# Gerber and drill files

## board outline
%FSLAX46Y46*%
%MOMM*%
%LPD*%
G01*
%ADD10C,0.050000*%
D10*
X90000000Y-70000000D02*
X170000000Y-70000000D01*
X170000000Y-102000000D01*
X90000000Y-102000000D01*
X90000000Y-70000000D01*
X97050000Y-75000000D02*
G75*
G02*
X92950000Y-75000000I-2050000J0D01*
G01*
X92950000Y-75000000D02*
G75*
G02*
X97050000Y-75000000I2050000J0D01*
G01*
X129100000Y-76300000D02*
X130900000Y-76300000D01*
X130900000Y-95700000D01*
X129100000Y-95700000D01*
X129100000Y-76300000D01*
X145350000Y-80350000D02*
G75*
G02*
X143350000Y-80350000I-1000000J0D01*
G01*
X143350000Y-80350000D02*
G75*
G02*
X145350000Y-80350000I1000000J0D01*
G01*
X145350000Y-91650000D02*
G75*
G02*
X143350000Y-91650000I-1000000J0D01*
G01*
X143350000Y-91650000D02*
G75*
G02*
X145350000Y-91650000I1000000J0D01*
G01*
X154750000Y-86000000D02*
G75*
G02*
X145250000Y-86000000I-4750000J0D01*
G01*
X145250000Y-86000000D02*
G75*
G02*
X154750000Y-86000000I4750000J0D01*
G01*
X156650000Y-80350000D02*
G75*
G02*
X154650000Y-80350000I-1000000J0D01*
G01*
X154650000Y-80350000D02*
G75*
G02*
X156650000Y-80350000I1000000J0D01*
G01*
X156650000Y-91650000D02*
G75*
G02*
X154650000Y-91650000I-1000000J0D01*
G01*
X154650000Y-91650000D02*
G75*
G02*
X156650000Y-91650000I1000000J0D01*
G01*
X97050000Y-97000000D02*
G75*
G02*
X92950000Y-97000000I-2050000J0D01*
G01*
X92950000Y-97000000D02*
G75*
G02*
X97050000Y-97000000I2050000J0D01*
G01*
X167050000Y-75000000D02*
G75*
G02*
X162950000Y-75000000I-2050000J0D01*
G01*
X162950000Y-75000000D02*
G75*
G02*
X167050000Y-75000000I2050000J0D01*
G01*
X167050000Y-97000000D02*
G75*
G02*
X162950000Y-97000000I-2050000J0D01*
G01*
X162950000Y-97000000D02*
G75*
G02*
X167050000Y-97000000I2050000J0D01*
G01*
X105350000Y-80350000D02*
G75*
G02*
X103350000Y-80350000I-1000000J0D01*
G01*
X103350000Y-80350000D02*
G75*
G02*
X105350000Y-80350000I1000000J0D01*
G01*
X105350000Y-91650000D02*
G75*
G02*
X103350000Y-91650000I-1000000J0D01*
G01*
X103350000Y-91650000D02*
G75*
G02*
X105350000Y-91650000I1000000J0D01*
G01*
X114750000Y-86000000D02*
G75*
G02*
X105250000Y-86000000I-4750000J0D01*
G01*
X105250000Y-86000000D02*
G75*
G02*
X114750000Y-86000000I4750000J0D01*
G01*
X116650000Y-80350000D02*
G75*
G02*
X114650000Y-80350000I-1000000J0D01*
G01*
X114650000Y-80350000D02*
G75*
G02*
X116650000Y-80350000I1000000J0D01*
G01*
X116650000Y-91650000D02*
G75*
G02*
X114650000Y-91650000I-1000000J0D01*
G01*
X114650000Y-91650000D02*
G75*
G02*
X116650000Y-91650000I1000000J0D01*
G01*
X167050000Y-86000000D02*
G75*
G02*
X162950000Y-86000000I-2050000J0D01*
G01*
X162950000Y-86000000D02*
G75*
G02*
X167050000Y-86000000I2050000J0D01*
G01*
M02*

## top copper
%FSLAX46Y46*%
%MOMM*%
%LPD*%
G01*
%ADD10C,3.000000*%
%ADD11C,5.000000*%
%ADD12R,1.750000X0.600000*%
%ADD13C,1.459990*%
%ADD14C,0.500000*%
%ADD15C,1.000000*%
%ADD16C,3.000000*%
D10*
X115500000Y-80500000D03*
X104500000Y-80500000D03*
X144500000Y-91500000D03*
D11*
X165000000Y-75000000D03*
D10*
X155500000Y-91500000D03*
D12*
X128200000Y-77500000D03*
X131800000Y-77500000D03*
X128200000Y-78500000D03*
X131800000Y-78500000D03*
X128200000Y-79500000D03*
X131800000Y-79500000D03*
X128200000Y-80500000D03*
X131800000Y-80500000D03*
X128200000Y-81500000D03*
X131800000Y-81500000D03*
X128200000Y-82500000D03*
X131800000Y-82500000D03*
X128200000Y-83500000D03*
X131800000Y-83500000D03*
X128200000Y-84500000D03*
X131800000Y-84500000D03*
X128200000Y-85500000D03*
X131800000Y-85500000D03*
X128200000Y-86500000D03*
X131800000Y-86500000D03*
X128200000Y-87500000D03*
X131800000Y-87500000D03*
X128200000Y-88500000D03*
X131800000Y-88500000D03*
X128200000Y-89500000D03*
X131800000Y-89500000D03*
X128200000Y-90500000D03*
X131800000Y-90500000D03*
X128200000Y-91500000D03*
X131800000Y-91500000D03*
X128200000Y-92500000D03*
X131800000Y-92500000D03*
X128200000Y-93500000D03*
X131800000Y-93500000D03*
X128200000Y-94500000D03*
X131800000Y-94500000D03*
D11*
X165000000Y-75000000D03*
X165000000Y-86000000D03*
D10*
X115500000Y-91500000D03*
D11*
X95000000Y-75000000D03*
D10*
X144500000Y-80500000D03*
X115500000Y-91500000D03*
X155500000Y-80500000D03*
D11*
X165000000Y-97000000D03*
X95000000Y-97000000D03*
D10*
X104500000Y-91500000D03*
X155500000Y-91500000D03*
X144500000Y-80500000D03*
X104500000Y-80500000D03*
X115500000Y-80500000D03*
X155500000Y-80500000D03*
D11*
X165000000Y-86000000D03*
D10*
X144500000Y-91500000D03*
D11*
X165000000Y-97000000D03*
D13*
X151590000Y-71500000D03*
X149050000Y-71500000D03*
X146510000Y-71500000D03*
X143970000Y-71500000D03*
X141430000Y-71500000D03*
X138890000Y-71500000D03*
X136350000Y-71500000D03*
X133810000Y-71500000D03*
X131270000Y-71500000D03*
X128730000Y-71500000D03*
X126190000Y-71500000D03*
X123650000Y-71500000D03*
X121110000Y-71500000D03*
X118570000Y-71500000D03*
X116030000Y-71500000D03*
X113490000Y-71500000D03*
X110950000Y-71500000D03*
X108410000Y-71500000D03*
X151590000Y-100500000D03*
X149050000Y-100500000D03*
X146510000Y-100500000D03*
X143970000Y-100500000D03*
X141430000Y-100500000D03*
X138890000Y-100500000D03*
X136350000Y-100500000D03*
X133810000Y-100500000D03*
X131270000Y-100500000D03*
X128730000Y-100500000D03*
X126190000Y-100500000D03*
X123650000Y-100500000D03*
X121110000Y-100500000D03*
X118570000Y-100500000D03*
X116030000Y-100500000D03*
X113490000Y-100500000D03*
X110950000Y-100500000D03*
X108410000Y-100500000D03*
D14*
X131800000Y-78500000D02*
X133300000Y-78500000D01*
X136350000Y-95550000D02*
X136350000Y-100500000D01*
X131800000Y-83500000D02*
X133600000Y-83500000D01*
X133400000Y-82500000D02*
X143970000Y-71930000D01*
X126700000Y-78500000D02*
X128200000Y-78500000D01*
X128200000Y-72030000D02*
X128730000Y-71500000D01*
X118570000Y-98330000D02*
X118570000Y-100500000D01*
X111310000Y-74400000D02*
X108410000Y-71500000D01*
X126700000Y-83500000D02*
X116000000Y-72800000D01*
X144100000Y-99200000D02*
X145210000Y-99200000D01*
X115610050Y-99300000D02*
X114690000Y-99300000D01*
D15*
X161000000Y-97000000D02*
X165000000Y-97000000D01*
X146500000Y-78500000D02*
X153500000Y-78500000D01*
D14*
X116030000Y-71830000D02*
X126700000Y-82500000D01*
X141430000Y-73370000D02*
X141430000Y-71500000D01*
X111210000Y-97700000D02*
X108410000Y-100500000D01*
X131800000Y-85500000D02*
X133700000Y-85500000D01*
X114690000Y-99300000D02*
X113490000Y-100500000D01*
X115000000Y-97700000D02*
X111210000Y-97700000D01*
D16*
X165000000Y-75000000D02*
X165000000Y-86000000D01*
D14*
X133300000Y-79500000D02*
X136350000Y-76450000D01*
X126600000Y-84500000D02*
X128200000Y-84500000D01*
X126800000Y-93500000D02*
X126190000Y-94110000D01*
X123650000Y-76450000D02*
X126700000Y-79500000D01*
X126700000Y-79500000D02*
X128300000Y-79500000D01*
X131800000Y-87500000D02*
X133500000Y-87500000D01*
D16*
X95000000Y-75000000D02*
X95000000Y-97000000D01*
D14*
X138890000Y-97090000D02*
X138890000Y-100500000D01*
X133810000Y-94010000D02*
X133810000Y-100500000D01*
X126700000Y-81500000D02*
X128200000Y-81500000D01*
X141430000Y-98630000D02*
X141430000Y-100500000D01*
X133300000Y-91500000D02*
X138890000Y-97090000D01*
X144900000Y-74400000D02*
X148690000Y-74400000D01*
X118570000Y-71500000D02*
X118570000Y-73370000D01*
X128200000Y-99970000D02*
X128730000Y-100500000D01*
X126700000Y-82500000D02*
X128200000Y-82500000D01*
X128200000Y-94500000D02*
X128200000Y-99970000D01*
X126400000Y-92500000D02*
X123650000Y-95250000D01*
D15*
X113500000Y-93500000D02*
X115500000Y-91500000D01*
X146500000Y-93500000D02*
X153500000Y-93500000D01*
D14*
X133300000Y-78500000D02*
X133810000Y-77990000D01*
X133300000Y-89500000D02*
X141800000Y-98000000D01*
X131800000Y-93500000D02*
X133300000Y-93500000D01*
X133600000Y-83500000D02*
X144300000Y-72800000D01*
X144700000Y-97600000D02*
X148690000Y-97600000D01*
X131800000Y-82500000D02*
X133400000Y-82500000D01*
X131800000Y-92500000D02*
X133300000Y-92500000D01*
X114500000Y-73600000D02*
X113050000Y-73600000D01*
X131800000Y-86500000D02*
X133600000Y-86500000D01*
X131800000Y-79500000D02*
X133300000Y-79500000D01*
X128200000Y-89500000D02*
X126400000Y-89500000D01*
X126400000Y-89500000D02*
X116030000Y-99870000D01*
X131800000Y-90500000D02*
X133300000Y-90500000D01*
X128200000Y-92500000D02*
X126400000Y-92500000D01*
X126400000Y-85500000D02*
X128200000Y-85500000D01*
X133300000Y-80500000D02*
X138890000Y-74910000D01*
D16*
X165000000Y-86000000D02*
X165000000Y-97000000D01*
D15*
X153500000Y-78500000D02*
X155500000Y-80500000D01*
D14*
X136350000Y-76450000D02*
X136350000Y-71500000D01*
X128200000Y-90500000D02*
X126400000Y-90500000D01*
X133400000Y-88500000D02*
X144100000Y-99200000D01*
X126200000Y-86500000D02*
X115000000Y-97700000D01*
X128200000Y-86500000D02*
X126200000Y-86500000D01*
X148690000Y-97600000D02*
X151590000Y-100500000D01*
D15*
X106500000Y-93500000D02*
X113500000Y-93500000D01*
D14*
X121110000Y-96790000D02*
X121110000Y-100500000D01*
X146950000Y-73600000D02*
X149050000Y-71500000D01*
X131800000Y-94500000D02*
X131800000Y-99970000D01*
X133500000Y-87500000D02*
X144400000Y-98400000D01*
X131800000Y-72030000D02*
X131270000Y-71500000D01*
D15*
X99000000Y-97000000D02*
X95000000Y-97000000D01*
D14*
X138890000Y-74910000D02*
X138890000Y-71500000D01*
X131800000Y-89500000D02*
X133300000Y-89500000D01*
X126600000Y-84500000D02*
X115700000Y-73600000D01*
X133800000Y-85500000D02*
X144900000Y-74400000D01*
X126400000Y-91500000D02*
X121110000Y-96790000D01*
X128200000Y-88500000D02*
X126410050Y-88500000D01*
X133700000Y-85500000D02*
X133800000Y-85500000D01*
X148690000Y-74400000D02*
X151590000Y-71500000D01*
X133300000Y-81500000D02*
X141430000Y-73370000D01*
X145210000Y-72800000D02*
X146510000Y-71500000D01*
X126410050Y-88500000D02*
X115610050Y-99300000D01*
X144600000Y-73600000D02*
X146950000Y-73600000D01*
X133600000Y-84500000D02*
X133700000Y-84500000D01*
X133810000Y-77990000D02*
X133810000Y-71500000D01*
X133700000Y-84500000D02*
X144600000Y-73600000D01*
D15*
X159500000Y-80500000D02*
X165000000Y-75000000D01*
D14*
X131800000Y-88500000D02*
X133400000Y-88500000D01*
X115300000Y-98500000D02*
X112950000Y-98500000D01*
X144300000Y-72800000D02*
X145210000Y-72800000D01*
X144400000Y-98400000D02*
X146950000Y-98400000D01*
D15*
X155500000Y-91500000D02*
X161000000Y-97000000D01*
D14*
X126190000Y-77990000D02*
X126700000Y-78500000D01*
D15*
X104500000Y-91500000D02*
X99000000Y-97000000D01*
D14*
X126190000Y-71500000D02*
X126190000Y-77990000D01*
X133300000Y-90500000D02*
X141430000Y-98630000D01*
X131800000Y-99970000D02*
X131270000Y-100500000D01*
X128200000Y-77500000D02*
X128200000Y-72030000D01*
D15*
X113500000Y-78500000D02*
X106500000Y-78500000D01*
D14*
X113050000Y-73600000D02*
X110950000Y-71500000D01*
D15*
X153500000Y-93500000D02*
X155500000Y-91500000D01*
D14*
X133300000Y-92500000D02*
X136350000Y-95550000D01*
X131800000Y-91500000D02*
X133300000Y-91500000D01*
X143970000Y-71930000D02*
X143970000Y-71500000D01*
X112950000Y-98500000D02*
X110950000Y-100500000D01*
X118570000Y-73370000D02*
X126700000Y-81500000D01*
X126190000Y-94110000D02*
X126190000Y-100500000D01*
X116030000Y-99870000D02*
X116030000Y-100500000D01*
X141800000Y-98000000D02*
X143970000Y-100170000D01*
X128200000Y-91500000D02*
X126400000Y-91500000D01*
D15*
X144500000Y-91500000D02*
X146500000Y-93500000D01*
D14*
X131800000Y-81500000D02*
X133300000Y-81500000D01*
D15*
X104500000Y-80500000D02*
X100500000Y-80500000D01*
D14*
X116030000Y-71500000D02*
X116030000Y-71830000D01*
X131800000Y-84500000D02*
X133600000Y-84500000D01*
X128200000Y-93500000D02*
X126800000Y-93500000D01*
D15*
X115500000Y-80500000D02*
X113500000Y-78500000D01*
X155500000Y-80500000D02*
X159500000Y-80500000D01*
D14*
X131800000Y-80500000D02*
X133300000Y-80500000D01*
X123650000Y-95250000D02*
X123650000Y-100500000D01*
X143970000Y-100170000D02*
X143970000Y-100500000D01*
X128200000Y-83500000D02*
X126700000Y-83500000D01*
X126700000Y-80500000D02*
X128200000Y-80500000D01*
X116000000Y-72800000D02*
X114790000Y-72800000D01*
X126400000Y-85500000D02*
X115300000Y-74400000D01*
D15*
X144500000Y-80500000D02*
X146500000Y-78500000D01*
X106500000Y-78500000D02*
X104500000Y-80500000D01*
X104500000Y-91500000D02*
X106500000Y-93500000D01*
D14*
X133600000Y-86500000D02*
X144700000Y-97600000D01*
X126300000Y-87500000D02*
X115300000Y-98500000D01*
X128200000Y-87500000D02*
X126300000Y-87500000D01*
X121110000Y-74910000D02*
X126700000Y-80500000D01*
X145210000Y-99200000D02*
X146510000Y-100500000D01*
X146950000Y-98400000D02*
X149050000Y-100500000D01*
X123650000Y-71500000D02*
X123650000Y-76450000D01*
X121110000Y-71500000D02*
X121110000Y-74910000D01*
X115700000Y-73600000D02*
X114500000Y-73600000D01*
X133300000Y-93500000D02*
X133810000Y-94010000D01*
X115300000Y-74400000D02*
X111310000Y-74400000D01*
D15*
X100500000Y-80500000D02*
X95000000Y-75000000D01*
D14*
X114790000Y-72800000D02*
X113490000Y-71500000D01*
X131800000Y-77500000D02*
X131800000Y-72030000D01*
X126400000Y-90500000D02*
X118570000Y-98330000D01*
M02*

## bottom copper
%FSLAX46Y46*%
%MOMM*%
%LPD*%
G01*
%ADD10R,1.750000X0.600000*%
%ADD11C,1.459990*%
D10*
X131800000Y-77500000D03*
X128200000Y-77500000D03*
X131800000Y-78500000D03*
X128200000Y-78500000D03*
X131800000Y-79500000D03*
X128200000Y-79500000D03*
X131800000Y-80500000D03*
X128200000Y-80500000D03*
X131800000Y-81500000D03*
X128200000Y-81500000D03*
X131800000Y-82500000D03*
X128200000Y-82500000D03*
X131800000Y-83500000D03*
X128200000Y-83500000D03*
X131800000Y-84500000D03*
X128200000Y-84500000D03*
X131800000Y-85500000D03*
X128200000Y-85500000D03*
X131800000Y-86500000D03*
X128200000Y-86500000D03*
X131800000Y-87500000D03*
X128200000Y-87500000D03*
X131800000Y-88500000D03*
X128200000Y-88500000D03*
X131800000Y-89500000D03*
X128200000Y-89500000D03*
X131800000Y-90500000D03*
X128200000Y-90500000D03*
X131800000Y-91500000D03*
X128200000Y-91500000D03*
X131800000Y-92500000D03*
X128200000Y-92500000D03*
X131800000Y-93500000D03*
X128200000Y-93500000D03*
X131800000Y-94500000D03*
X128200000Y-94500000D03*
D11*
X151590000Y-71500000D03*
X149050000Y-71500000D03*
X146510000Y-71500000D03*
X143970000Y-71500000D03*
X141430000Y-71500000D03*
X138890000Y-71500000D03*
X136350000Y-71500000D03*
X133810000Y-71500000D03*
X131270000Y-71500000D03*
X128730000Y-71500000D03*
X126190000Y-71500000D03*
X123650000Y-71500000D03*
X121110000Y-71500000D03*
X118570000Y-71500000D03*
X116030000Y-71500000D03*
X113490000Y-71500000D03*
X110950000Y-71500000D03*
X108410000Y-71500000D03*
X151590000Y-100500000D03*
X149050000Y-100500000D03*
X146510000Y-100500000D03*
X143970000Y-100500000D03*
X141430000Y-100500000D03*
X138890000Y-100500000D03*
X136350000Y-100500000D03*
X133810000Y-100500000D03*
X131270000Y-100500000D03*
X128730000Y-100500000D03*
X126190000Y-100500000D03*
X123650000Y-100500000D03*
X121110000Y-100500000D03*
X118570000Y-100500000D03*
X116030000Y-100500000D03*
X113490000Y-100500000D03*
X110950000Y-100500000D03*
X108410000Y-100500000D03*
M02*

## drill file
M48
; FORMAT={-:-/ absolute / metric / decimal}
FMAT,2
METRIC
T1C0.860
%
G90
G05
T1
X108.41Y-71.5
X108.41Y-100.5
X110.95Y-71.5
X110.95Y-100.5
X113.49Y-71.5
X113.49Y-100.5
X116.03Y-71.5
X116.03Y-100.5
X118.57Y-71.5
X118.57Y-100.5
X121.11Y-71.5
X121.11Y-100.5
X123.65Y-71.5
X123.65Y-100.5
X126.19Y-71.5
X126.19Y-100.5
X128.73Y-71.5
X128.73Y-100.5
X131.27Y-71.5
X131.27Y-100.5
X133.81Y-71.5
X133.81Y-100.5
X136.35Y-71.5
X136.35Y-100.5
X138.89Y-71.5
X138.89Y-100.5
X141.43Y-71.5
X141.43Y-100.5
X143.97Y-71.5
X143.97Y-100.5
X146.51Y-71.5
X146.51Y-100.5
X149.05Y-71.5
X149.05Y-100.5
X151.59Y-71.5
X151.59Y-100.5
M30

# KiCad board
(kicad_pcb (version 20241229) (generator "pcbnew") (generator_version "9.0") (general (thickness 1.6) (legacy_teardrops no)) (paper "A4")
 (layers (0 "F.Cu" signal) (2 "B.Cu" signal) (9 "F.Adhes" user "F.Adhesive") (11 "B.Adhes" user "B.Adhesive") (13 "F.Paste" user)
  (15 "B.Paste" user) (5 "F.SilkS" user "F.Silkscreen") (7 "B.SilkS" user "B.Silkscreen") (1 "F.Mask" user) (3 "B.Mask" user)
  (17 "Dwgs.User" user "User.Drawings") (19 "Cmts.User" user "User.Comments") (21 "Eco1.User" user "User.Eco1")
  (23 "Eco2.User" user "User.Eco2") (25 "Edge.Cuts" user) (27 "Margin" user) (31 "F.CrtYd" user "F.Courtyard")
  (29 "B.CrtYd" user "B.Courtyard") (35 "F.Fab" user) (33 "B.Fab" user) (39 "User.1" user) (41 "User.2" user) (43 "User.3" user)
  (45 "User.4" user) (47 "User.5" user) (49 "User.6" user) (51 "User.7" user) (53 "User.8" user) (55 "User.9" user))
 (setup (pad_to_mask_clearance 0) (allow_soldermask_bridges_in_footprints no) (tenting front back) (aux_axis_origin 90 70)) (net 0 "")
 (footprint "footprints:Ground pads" (layer "F.Cu") (at 115.5 80.5)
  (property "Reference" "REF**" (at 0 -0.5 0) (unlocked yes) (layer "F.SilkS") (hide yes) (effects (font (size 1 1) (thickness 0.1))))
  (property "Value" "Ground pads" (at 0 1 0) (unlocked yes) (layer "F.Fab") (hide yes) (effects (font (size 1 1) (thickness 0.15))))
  (pad "1" smd circle (at 0 0) (size 3 3) (layers "F.Cu" "F.Mask" "F.Paste")))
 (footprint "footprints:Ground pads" (layer "F.Cu") (at 104.5 80.5)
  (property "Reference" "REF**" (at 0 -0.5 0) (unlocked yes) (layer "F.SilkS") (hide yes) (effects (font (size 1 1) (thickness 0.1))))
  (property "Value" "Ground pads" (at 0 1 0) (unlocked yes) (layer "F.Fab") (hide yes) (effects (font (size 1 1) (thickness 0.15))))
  (pad "1" smd circle (at 0 0) (size 3 3) (layers "F.Cu" "F.Mask" "F.Paste")))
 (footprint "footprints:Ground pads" (layer "F.Cu") (at 144.5 91.5)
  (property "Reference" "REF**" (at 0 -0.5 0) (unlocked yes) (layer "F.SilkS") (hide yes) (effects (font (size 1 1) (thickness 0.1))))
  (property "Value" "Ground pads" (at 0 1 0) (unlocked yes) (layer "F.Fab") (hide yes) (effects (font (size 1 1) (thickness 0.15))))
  (pad "1" smd circle (at 0 0) (size 3 3) (layers "F.Cu" "F.Mask" "F.Paste")))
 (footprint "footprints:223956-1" (layer "F.Cu") (at 95 75)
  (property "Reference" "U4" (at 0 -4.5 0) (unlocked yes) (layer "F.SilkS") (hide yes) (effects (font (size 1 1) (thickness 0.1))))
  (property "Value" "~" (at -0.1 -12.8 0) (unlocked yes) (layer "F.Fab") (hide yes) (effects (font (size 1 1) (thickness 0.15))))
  (fp_circle (center 0 0) (end 0 2.05) (stroke (width 0.05) (type default)) (fill no) (layer "Edge.Cuts")))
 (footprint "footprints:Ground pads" (layer "F.Cu") (at 165 75)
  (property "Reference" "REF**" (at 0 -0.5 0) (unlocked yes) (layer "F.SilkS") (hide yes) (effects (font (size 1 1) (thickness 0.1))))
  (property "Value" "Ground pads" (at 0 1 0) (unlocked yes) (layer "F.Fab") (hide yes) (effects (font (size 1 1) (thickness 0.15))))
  (pad "1" smd circle (at 0 0) (size 5 5) (layers "F.Cu" "F.Mask" "F.Paste")))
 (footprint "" (layer "F.Cu") (at 155.5 91.5)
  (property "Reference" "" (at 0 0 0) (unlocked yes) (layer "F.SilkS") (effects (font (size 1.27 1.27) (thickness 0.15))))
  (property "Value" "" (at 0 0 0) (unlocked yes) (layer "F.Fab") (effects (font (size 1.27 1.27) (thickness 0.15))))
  (pad "1" smd circle (at 0 0) (size 3 3) (layers "F.Cu" "F.Mask" "F.Paste")))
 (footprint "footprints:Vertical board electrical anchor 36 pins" (layer "F.Cu") (at 130 86)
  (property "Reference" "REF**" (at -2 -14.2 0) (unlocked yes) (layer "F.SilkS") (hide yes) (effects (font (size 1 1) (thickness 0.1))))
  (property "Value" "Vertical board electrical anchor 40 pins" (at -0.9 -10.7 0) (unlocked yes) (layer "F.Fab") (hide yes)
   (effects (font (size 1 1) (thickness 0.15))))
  (fp_rect (start -0.9 -9.7) (end 0.9 9.7) (stroke (width 0.05) (type default)) (fill no) (layer "Edge.Cuts"))
  (pad "01A" smd rect (at -1.8 -8.5 90) (size 0.6 1.75) (layers "F.Cu" "F.Mask" "F.Paste") (solder_mask_margin 0.102))
  (pad "01A" smd rect (at 1.8 -8.5 90) (size 0.6 1.75) (layers "F.Cu" "F.Mask" "F.Paste") (solder_mask_margin 0.102))
  (pad "02A" smd rect (at -1.8 -7.5 90) (size 0.6 1.75) (layers "F.Cu" "F.Mask" "F.Paste") (solder_mask_margin 0.102))
  (pad "02A" smd rect (at 1.8 -7.5 90) (size 0.6 1.75) (layers "F.Cu" "F.Mask" "F.Paste") (solder_mask_margin 0.102))
  (pad "03A" smd rect (at -1.8 -6.5 90) (size 0.6 1.75) (layers "F.Cu" "F.Mask" "F.Paste") (solder_mask_margin 0.102))
  (pad "03A" smd rect (at 1.8 -6.5 90) (size 0.6 1.75) (layers "F.Cu" "F.Mask" "F.Paste") (solder_mask_margin 0.102))
  (pad "04A" smd rect (at -1.8 -5.5 90) (size 0.6 1.75) (layers "F.Cu" "F.Mask" "F.Paste") (solder_mask_margin 0.102))
  (pad "04A" smd rect (at 1.8 -5.5 90) (size 0.6 1.75) (layers "F.Cu" "F.Mask" "F.Paste") (solder_mask_margin 0.102))
  (pad "05A" smd rect (at -1.8 -4.5 90) (size 0.6 1.75) (layers "F.Cu" "F.Mask" "F.Paste") (solder_mask_margin 0.102))
  (pad "05A" smd rect (at 1.8 -4.5 90) (size 0.6 1.75) (layers "F.Cu" "F.Mask" "F.Paste") (solder_mask_margin 0.102))
  (pad "06A" smd rect (at -1.8 -3.5 90) (size 0.6 1.75) (layers "F.Cu" "F.Mask" "F.Paste") (solder_mask_margin 0.102))
  (pad "06A" smd rect (at 1.8 -3.5 90) (size 0.6 1.75) (layers "F.Cu" "F.Mask" "F.Paste") (solder_mask_margin 0.102))
  (pad "07A" smd rect (at -1.8 -2.5 90) (size 0.6 1.75) (layers "F.Cu" "F.Mask" "F.Paste") (solder_mask_margin 0.102))
  (pad "07A" smd rect (at 1.8 -2.5 90) (size 0.6 1.75) (layers "F.Cu" "F.Mask" "F.Paste") (solder_mask_margin 0.102))
  (pad "08A" smd rect (at -1.8 -1.5 90) (size 0.6 1.75) (layers "F.Cu" "F.Mask" "F.Paste") (solder_mask_margin 0.102))
  (pad "08A" smd rect (at 1.8 -1.5 90) (size 0.6 1.75) (layers "F.Cu" "F.Mask" "F.Paste") (solder_mask_margin 0.102))
  (pad "09A" smd rect (at -1.8 -0.5 90) (size 0.6 1.75) (layers "F.Cu" "F.Mask" "F.Paste") (solder_mask_margin 0.102))
  (pad "09A" smd rect (at 1.8 -0.5 90) (size 0.6 1.75) (layers "F.Cu" "F.Mask" "F.Paste") (solder_mask_margin 0.102))
  (pad "10A" smd rect (at -1.8 0.5 90) (size 0.6 1.75) (layers "F.Cu" "F.Mask" "F.Paste") (solder_mask_margin 0.102))
  (pad "10A" smd rect (at 1.8 0.5 90) (size 0.6 1.75) (layers "F.Cu" "F.Mask" "F.Paste") (solder_mask_margin 0.102))
  (pad "11A" smd rect (at -1.8 1.5 90) (size 0.6 1.75) (layers "F.Cu" "F.Mask" "F.Paste") (solder_mask_margin 0.102))
  (pad "11A" smd rect (at 1.8 1.5 90) (size 0.6 1.75) (layers "F.Cu" "F.Mask" "F.Paste") (solder_mask_margin 0.102))
  (pad "12A" smd rect (at -1.8 2.5 90) (size 0.6 1.75) (layers "F.Cu" "F.Mask" "F.Paste") (solder_mask_margin 0.102))
  (pad "12A" smd rect (at 1.8 2.5 90) (size 0.6 1.75) (layers "F.Cu" "F.Mask" "F.Paste") (solder_mask_margin 0.102))
  (pad "13A" smd rect (at -1.8 3.5 90) (size 0.6 1.75) (layers "F.Cu" "F.Mask" "F.Paste") (solder_mask_margin 0.102))
  (pad "13A" smd rect (at 1.8 3.5 90) (size 0.6 1.75) (layers "F.Cu" "F.Mask" "F.Paste") (solder_mask_margin 0.102))
  (pad "14A" smd rect (at -1.8 4.5 90) (size 0.6 1.75) (layers "F.Cu" "F.Mask" "F.Paste") (solder_mask_margin 0.102))
  (pad "14A" smd rect (at 1.8 4.5 90) (size 0.6 1.75) (layers "F.Cu" "F.Mask" "F.Paste") (solder_mask_margin 0.102))
  (pad "15A" smd rect (at -1.8 5.5 90) (size 0.6 1.75) (layers "F.Cu" "F.Mask" "F.Paste") (solder_mask_margin 0.102))
  (pad "15A" smd rect (at 1.8 5.5 90) (size 0.6 1.75) (layers "F.Cu" "F.Mask" "F.Paste") (solder_mask_margin 0.102))
  (pad "16A" smd rect (at -1.8 6.5 90) (size 0.6 1.75) (layers "F.Cu" "F.Mask" "F.Paste") (solder_mask_margin 0.102))
  (pad "16A" smd rect (at 1.8 6.5 90) (size 0.6 1.75) (layers "F.Cu" "F.Mask" "F.Paste") (solder_mask_margin 0.102))
  (pad "17A" smd rect (at -1.8 7.5 90) (size 0.6 1.75) (layers "F.Cu" "F.Mask" "F.Paste") (solder_mask_margin 0.102))
  (pad "17A" smd rect (at 1.8 7.5 90) (size 0.6 1.75) (layers "F.Cu" "F.Mask" "F.Paste") (solder_mask_margin 0.102))
  (pad "18A" smd rect (at -1.8 8.5 90) (size 0.6 1.75) (layers "F.Cu" "F.Mask" "F.Paste") (solder_mask_margin 0.102))
  (pad "18A" smd rect (at 1.8 8.5 90) (size 0.6 1.75) (layers "F.Cu" "F.Mask" "F.Paste") (solder_mask_margin 0.102)))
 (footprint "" (layer "F.Cu") (at 165 75)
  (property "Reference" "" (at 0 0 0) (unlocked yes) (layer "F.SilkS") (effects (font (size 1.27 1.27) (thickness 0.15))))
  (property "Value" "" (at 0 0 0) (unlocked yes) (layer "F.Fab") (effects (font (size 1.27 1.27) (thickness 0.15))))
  (pad "1" smd circle (at 0 0) (size 5 5) (layers "F.Cu" "F.Mask" "F.Paste")))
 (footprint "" (layer "F.Cu") (at 165 86)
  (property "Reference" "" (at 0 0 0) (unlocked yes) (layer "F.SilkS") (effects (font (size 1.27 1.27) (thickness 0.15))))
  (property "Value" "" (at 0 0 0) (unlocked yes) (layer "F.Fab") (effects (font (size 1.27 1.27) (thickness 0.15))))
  (pad "1" smd circle (at 0 0) (size 5 5) (layers "F.Cu" "F.Mask" "F.Paste")))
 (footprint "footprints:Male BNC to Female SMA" (layer "F.Cu") (at 150 86)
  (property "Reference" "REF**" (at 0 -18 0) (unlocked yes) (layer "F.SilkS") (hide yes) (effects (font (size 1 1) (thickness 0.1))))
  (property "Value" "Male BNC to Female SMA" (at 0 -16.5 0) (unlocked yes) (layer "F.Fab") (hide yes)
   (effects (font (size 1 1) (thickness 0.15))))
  (fp_circle (center -5.65 -5.65) (end -5.65 -4.65) (stroke (width 0.05) (type default)) (fill no) (layer "Edge.Cuts"))
  (fp_circle (center -5.65 5.65) (end -5.65 6.65) (stroke (width 0.05) (type default)) (fill no) (layer "Edge.Cuts"))
  (fp_circle (center 0 0) (end 0 -4.75) (stroke (width 0.05) (type default)) (fill no) (layer "Edge.Cuts"))
  (fp_circle (center 5.65 -5.65) (end 5.65 -6.65) (stroke (width 0.05) (type default)) (fill no) (layer "Edge.Cuts"))
  (fp_circle (center 5.65 5.65) (end 4.65 5.65) (stroke (width 0.05) (type default)) (fill no) (layer "Edge.Cuts")))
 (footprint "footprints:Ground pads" (layer "F.Cu") (at 115.5 91.5)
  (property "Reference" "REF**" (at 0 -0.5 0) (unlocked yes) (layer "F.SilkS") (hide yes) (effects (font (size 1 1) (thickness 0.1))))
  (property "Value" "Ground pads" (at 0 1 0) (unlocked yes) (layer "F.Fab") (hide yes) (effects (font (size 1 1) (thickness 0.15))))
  (pad "1" smd circle (at 0 0) (size 3 3) (layers "F.Cu" "F.Mask" "F.Paste")))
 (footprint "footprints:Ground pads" (layer "F.Cu") (at 95 75)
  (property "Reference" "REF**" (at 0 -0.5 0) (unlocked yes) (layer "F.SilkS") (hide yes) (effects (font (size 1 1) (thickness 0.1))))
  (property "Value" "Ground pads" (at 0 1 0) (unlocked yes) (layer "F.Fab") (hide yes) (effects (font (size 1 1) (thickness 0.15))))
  (pad "1" smd circle (at 0 0) (size 5 5) (layers "F.Cu" "F.Mask" "F.Paste")))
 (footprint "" (layer "F.Cu") (at 144.5 80.5)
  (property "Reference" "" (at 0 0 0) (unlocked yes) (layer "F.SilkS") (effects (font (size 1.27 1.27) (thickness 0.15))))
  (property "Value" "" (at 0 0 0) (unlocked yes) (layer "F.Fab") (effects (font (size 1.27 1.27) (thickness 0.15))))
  (pad "1" smd circle (at 0 0) (size 3 3) (layers "F.Cu" "F.Mask" "F.Paste")))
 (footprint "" (layer "F.Cu") (at 115.5 91.5)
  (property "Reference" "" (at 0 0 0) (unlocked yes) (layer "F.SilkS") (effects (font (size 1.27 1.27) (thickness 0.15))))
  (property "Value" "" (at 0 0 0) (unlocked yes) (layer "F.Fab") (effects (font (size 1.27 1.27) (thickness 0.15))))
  (pad "1" smd circle (at 0 0) (size 3 3) (layers "F.Cu" "F.Mask" "F.Paste")))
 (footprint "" (layer "F.Cu") (at 155.5 80.5)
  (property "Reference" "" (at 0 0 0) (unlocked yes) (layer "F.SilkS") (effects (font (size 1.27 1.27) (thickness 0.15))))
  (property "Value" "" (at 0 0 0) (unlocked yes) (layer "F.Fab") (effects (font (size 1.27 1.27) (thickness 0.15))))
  (pad "1" smd circle (at 0 0) (size 3 3) (layers "F.Cu" "F.Mask" "F.Paste")))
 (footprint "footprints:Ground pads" (layer "F.Cu") (at 165 97)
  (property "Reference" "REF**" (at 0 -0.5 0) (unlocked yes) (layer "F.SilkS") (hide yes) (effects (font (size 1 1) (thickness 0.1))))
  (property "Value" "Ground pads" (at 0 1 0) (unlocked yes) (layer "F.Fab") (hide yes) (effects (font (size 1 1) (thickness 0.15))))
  (pad "1" smd circle (at 0 0) (size 5 5) (layers "F.Cu" "F.Mask" "F.Paste")))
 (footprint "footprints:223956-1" (layer "F.Cu") (at 95 97)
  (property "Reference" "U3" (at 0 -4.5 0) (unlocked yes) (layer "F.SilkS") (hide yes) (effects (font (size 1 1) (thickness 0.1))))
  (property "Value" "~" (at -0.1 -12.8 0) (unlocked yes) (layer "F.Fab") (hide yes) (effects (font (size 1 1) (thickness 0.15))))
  (fp_circle (center 0 0) (end 0 2.05) (stroke (width 0.05) (type default)) (fill no) (layer "Edge.Cuts")))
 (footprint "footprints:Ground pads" (layer "F.Cu") (at 95 97)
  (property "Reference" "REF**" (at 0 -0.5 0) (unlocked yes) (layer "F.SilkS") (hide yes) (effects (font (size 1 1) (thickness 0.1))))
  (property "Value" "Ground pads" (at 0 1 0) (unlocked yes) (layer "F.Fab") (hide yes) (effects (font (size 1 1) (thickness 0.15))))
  (pad "1" smd circle (at 0 0) (size 5 5) (layers "F.Cu" "F.Mask" "F.Paste")))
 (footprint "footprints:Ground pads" (layer "F.Cu") (at 104.5 91.5)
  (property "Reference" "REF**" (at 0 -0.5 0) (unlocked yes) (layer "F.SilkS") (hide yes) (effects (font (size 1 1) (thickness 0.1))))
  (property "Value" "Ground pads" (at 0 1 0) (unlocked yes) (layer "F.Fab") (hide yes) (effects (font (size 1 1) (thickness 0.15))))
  (pad "1" smd circle (at 0 0) (size 3 3) (layers "F.Cu" "F.Mask" "F.Paste")))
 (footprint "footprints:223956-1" (layer "F.Cu") (at 165 75)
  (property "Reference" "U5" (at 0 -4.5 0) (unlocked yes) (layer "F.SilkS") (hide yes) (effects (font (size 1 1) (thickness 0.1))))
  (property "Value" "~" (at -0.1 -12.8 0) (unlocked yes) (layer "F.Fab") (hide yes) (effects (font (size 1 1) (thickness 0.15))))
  (fp_circle (center 0 0) (end 0 2.05) (stroke (width 0.05) (type default)) (fill no) (layer "Edge.Cuts")))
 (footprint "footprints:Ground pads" (layer "F.Cu") (at 155.5 91.5)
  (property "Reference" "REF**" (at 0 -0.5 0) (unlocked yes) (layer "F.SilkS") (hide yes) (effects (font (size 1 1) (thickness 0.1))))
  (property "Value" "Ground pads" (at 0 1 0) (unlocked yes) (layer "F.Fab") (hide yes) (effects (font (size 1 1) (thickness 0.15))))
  (pad "1" smd circle (at 0 0) (size 3 3) (layers "F.Cu" "F.Mask" "F.Paste")))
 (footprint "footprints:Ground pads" (layer "F.Cu") (at 144.5 80.5)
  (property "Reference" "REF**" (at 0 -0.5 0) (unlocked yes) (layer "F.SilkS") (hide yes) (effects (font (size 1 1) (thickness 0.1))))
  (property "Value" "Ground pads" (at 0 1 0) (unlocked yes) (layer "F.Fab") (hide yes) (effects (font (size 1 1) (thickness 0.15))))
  (pad "1" smd circle (at 0 0) (size 3 3) (layers "F.Cu" "F.Mask" "F.Paste")))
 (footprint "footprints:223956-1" (layer "F.Cu") (at 165 97)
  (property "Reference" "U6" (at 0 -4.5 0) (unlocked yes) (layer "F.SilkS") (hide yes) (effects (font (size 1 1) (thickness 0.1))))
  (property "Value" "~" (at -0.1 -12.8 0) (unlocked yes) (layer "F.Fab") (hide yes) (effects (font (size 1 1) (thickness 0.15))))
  (fp_circle (center 0 0) (end 0 2.05) (stroke (width 0.05) (type default)) (fill no) (layer "Edge.Cuts")))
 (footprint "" (layer "F.Cu") (at 104.5 80.5)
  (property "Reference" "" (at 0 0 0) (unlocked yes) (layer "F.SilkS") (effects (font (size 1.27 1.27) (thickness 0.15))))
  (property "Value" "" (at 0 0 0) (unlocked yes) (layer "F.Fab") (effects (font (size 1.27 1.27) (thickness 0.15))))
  (pad "1" smd circle (at 0 0) (size 3 3) (layers "F.Cu" "F.Mask" "F.Paste")))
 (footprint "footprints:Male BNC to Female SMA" (layer "F.Cu") (at 110 86)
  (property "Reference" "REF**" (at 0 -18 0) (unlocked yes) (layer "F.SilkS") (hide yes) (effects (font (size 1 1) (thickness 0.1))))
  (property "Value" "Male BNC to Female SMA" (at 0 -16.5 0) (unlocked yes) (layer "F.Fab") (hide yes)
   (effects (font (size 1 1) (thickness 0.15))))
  (fp_circle (center -5.65 -5.65) (end -5.65 -4.65) (stroke (width 0.05) (type default)) (fill no) (layer "Edge.Cuts"))
  (fp_circle (center -5.65 5.65) (end -5.65 6.65) (stroke (width 0.05) (type default)) (fill no) (layer "Edge.Cuts"))
  (fp_circle (center 0 0) (end 0 -4.75) (stroke (width 0.05) (type default)) (fill no) (layer "Edge.Cuts"))
  (fp_circle (center 5.65 -5.65) (end 5.65 -6.65) (stroke (width 0.05) (type default)) (fill no) (layer "Edge.Cuts"))
  (fp_circle (center 5.65 5.65) (end 4.65 5.65) (stroke (width 0.05) (type default)) (fill no) (layer "Edge.Cuts")))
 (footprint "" (layer "F.Cu") (at 115.5 80.5)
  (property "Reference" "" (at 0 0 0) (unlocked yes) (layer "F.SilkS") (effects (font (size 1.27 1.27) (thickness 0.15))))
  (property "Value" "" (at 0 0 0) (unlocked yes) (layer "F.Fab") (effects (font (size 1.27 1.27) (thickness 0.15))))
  (pad "1" smd circle (at 0 0) (size 3 3) (layers "F.Cu" "F.Mask" "F.Paste")))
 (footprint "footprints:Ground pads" (layer "F.Cu") (at 155.5 80.5)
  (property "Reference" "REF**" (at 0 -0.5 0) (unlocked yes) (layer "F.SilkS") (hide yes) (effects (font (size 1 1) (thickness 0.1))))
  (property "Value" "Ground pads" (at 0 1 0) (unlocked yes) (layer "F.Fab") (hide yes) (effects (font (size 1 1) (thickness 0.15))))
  (pad "1" smd circle (at 0 0) (size 3 3) (layers "F.Cu" "F.Mask" "F.Paste")))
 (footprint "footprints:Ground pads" (layer "F.Cu") (at 165 86)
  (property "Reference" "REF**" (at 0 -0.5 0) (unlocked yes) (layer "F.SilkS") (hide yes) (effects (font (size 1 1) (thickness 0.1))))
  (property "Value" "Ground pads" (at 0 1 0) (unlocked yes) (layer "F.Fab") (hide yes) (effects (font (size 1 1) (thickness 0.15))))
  (pad "1" smd circle (at 0 0) (size 5 5) (layers "F.Cu" "F.Mask" "F.Paste")))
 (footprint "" (layer "F.Cu") (at 144.5 91.5)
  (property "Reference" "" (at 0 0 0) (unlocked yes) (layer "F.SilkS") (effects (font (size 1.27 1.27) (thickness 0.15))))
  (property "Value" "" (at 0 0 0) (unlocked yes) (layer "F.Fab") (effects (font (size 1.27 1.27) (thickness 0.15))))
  (pad "1" smd circle (at 0 0) (size 3 3) (layers "F.Cu" "F.Mask" "F.Paste")))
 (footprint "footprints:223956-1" (layer "F.Cu") (at 165 86)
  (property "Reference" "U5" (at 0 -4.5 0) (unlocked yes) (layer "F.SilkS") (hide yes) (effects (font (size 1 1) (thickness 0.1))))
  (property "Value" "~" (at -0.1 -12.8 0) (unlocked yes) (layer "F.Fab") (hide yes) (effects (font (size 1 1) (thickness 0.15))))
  (fp_circle (center 0 0) (end 0 2.05) (stroke (width 0.05) (type default)) (fill no) (layer "Edge.Cuts")))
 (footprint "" (layer "F.Cu") (at 165 97)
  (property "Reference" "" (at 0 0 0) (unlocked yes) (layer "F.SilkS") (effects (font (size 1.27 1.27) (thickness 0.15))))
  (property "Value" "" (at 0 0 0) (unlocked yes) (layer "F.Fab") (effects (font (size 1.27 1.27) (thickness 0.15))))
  (pad "1" smd circle (at 0 0) (size 5 5) (layers "F.Cu" "F.Mask" "F.Paste")))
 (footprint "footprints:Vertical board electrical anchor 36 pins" (layer "B.Cu") (at 130 86 180)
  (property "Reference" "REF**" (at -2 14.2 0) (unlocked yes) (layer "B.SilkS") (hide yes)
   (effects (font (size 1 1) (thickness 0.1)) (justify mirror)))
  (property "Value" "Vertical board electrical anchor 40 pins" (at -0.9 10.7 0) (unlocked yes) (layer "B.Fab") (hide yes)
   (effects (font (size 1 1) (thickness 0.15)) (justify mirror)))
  (pad "01A" smd rect (at -1.8 8.5 90) (size 0.6 1.75) (layers "B.Cu" "B.Mask" "B.Paste") (solder_mask_margin 0.102))
  (pad "01A" smd rect (at 1.8 8.5 90) (size 0.6 1.75) (layers "B.Cu" "B.Mask" "B.Paste") (solder_mask_margin 0.102))
  (pad "02A" smd rect (at -1.8 7.5 90) (size 0.6 1.75) (layers "B.Cu" "B.Mask" "B.Paste") (solder_mask_margin 0.102))
  (pad "02A" smd rect (at 1.8 7.5 90) (size 0.6 1.75) (layers "B.Cu" "B.Mask" "B.Paste") (solder_mask_margin 0.102))
  (pad "03A" smd rect (at -1.8 6.5 90) (size 0.6 1.75) (layers "B.Cu" "B.Mask" "B.Paste") (solder_mask_margin 0.102))
  (pad "03A" smd rect (at 1.8 6.5 90) (size 0.6 1.75) (layers "B.Cu" "B.Mask" "B.Paste") (solder_mask_margin 0.102))
  (pad "04A" smd rect (at -1.8 5.5 90) (size 0.6 1.75) (layers "B.Cu" "B.Mask" "B.Paste") (solder_mask_margin 0.102))
  (pad "04A" smd rect (at 1.8 5.5 90) (size 0.6 1.75) (layers "B.Cu" "B.Mask" "B.Paste") (solder_mask_margin 0.102))
  (pad "05A" smd rect (at -1.8 4.5 90) (size 0.6 1.75) (layers "B.Cu" "B.Mask" "B.Paste") (solder_mask_margin 0.102))
  (pad "05A" smd rect (at 1.8 4.5 90) (size 0.6 1.75) (layers "B.Cu" "B.Mask" "B.Paste") (solder_mask_margin 0.102))
  (pad "06A" smd rect (at -1.8 3.5 90) (size 0.6 1.75) (layers "B.Cu" "B.Mask" "B.Paste") (solder_mask_margin 0.102))
  (pad "06A" smd rect (at 1.8 3.5 90) (size 0.6 1.75) (layers "B.Cu" "B.Mask" "B.Paste") (solder_mask_margin 0.102))
  (pad "07A" smd rect (at -1.8 2.5 90) (size 0.6 1.75) (layers "B.Cu" "B.Mask" "B.Paste") (solder_mask_margin 0.102))
  (pad "07A" smd rect (at 1.8 2.5 90) (size 0.6 1.75) (layers "B.Cu" "B.Mask" "B.Paste") (solder_mask_margin 0.102))
  (pad "08A" smd rect (at -1.8 1.5 90) (size 0.6 1.75) (layers "B.Cu" "B.Mask" "B.Paste") (solder_mask_margin 0.102))
  (pad "08A" smd rect (at 1.8 1.5 90) (size 0.6 1.75) (layers "B.Cu" "B.Mask" "B.Paste") (solder_mask_margin 0.102))
  (pad "09A" smd rect (at -1.8 0.5 90) (size 0.6 1.75) (layers "B.Cu" "B.Mask" "B.Paste") (solder_mask_margin 0.102))
  (pad "09A" smd rect (at 1.8 0.5 90) (size 0.6 1.75) (layers "B.Cu" "B.Mask" "B.Paste") (solder_mask_margin 0.102))
  (pad "10A" smd rect (at -1.8 -0.5 90) (size 0.6 1.75) (layers "B.Cu" "B.Mask" "B.Paste") (solder_mask_margin 0.102))
  (pad "10A" smd rect (at 1.8 -0.5 90) (size 0.6 1.75) (layers "B.Cu" "B.Mask" "B.Paste") (solder_mask_margin 0.102))
  (pad "11A" smd rect (at -1.8 -1.5 90) (size 0.6 1.75) (layers "B.Cu" "B.Mask" "B.Paste") (solder_mask_margin 0.102))
  (pad "11A" smd rect (at 1.8 -1.5 90) (size 0.6 1.75) (layers "B.Cu" "B.Mask" "B.Paste") (solder_mask_margin 0.102))
  (pad "12A" smd rect (at -1.8 -2.5 90) (size 0.6 1.75) (layers "B.Cu" "B.Mask" "B.Paste") (solder_mask_margin 0.102))
  (pad "12A" smd rect (at 1.8 -2.5 90) (size 0.6 1.75) (layers "B.Cu" "B.Mask" "B.Paste") (solder_mask_margin 0.102))
  (pad "13A" smd rect (at -1.8 -3.5 90) (size 0.6 1.75) (layers "B.Cu" "B.Mask" "B.Paste") (solder_mask_margin 0.102))
  (pad "13A" smd rect (at 1.8 -3.5 90) (size 0.6 1.75) (layers "B.Cu" "B.Mask" "B.Paste") (solder_mask_margin 0.102))
  (pad "14A" smd rect (at -1.8 -4.5 90) (size 0.6 1.75) (layers "B.Cu" "B.Mask" "B.Paste") (solder_mask_margin 0.102))
  (pad "14A" smd rect (at 1.8 -4.5 90) (size 0.6 1.75) (layers "B.Cu" "B.Mask" "B.Paste") (solder_mask_margin 0.102))
  (pad "15A" smd rect (at -1.8 -5.5 90) (size 0.6 1.75) (layers "B.Cu" "B.Mask" "B.Paste") (solder_mask_margin 0.102))
  (pad "15A" smd rect (at 1.8 -5.5 90) (size 0.6 1.75) (layers "B.Cu" "B.Mask" "B.Paste") (solder_mask_margin 0.102))
  (pad "16A" smd rect (at -1.8 -6.5 90) (size 0.6 1.75) (layers "B.Cu" "B.Mask" "B.Paste") (solder_mask_margin 0.102))
  (pad "16A" smd rect (at 1.8 -6.5 90) (size 0.6 1.75) (layers "B.Cu" "B.Mask" "B.Paste") (solder_mask_margin 0.102))
  (pad "17A" smd rect (at -1.8 -7.5 90) (size 0.6 1.75) (layers "B.Cu" "B.Mask" "B.Paste") (solder_mask_margin 0.102))
  (pad "17A" smd rect (at 1.8 -7.5 90) (size 0.6 1.75) (layers "B.Cu" "B.Mask" "B.Paste") (solder_mask_margin 0.102))
  (pad "18A" smd rect (at -1.8 -8.5 90) (size 0.6 1.75) (layers "B.Cu" "B.Mask" "B.Paste") (solder_mask_margin 0.102))
  (pad "18A" smd rect (at 1.8 -8.5 90) (size 0.6 1.75) (layers "B.Cu" "B.Mask" "B.Paste") (solder_mask_margin 0.102)))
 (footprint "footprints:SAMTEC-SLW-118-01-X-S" (layer "B.Cu") (at 130 71.5 180)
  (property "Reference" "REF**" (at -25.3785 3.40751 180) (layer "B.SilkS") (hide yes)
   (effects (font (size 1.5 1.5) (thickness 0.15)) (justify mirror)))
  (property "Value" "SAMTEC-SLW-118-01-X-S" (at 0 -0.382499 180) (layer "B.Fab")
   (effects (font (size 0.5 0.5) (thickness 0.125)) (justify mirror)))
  (pad "1" thru_hole circle (at -21.59 0 180) (size 1.45999 1.45999) (drill 0.859993) (layers "*.Cu") (remove_unused_layers no))
  (pad "2" thru_hole circle (at -19.05 0 180) (size 1.45999 1.45999) (drill 0.859993) (layers "*.Cu") (remove_unused_layers no))
  (pad "3" thru_hole circle (at -16.51 0 180) (size 1.45999 1.45999) (drill 0.859993) (layers "*.Cu") (remove_unused_layers no))
  (pad "4" thru_hole circle (at -13.97 0 180) (size 1.45999 1.45999) (drill 0.859993) (layers "*.Cu") (remove_unused_layers no))
  (pad "5" thru_hole circle (at -11.43 0 180) (size 1.45999 1.45999) (drill 0.859993) (layers "*.Cu") (remove_unused_layers no))
  (pad "6" thru_hole circle (at -8.89 0 180) (size 1.45999 1.45999) (drill 0.859993) (layers "*.Cu") (remove_unused_layers no))
  (pad "7" thru_hole circle (at -6.35 0 180) (size 1.45999 1.45999) (drill 0.859993) (layers "*.Cu") (remove_unused_layers no))
  (pad "8" thru_hole circle (at -3.81 0 180) (size 1.45999 1.45999) (drill 0.859993) (layers "*.Cu") (remove_unused_layers no))
  (pad "9" thru_hole circle (at -1.27 0 180) (size 1.45999 1.45999) (drill 0.859993) (layers "*.Cu") (remove_unused_layers no))
  (pad "10" thru_hole circle (at 1.27 0 180) (size 1.45999 1.45999) (drill 0.859993) (layers "*.Cu") (remove_unused_layers no))
  (pad "11" thru_hole circle (at 3.81 0 180) (size 1.45999 1.45999) (drill 0.859993) (layers "*.Cu") (remove_unused_layers no))
  (pad "12" thru_hole circle (at 6.35 0 180) (size 1.45999 1.45999) (drill 0.859993) (layers "*.Cu") (remove_unused_layers no))
  (pad "13" thru_hole circle (at 8.89 0 180) (size 1.45999 1.45999) (drill 0.859993) (layers "*.Cu") (remove_unused_layers no))
  (pad "14" thru_hole circle (at 11.43 0 180) (size 1.45999 1.45999) (drill 0.859993) (layers "*.Cu") (remove_unused_layers no))
  (pad "15" thru_hole circle (at 13.97 0 180) (size 1.45999 1.45999) (drill 0.859993) (layers "*.Cu") (remove_unused_layers no))
  (pad "16" thru_hole circle (at 16.51 0 180) (size 1.45999 1.45999) (drill 0.859993) (layers "*.Cu") (remove_unused_layers no))
  (pad "17" thru_hole circle (at 19.05 0 180) (size 1.45999 1.45999) (drill 0.859993) (layers "*.Cu") (remove_unused_layers no))
  (pad "18" thru_hole circle (at 21.59 0 180) (size 1.45999 1.45999) (drill 0.859993) (layers "*.Cu") (remove_unused_layers no)))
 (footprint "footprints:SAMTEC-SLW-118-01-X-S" (layer "B.Cu") (at 130 100.5 180)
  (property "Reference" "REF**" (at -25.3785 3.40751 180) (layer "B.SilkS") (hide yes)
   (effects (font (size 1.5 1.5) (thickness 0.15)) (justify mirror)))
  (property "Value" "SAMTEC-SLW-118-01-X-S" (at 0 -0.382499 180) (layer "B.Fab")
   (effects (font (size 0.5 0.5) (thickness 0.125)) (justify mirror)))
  (pad "1" thru_hole circle (at -21.59 0 180) (size 1.45999 1.45999) (drill 0.859993) (layers "*.Cu") (remove_unused_layers no))
  (pad "2" thru_hole circle (at -19.05 0 180) (size 1.45999 1.45999) (drill 0.859993) (layers "*.Cu") (remove_unused_layers no))
  (pad "3" thru_hole circle (at -16.51 0 180) (size 1.45999 1.45999) (drill 0.859993) (layers "*.Cu") (remove_unused_layers no))
  (pad "4" thru_hole circle (at -13.97 0 180) (size 1.45999 1.45999) (drill 0.859993) (layers "*.Cu") (remove_unused_layers no))
  (pad "5" thru_hole circle (at -11.43 0 180) (size 1.45999 1.45999) (drill 0.859993) (layers "*.Cu") (remove_unused_layers no))
  (pad "6" thru_hole circle (at -8.89 0 180) (size 1.45999 1.45999) (drill 0.859993) (layers "*.Cu") (remove_unused_layers no))
  (pad "7" thru_hole circle (at -6.35 0 180) (size 1.45999 1.45999) (drill 0.859993) (layers "*.Cu") (remove_unused_layers no))
  (pad "8" thru_hole circle (at -3.81 0 180) (size 1.45999 1.45999) (drill 0.859993) (layers "*.Cu") (remove_unused_layers no))
  (pad "9" thru_hole circle (at -1.27 0 180) (size 1.45999 1.45999) (drill 0.859993) (layers "*.Cu") (remove_unused_layers no))
  (pad "10" thru_hole circle (at 1.27 0 180) (size 1.45999 1.45999) (drill 0.859993) (layers "*.Cu") (remove_unused_layers no))
  (pad "11" thru_hole circle (at 3.81 0 180) (size 1.45999 1.45999) (drill 0.859993) (layers "*.Cu") (remove_unused_layers no))
  (pad "12" thru_hole circle (at 6.35 0 180) (size 1.45999 1.45999) (drill 0.859993) (layers "*.Cu") (remove_unused_layers no))
  (pad "13" thru_hole circle (at 8.89 0 180) (size 1.45999 1.45999) (drill 0.859993) (layers "*.Cu") (remove_unused_layers no))
  (pad "14" thru_hole circle (at 11.43 0 180) (size 1.45999 1.45999) (drill 0.859993) (layers "*.Cu") (remove_unused_layers no))
  (pad "15" thru_hole circle (at 13.97 0 180) (size 1.45999 1.45999) (drill 0.859993) (layers "*.Cu") (remove_unused_layers no))
  (pad "16" thru_hole circle (at 16.51 0 180) (size 1.45999 1.45999) (drill 0.859993) (layers "*.Cu") (remove_unused_layers no))
  (pad "17" thru_hole circle (at 19.05 0 180) (size 1.45999 1.45999) (drill 0.859993) (layers "*.Cu") (remove_unused_layers no))
  (pad "18" thru_hole circle (at 21.59 0 180) (size 1.45999 1.45999) (drill 0.859993) (layers "*.Cu") (remove_unused_layers no)))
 (gr_rect (start 90 70) (end 170 102) (stroke (width 0.05) (type default)) (fill no) (layer "Edge.Cuts"))
 (segment (start 131.8 78.5) (end 133.3 78.5) (width 0.5) (layer "F.Cu") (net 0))
 (segment (start 136.35 95.55) (end 136.35 100.5) (width 0.5) (layer "F.Cu") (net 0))
 (segment (start 131.8 83.5) (end 133.6 83.5) (width 0.5) (layer "F.Cu") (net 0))
 (segment (start 133.4 82.5) (end 143.97 71.93) (width 0.5) (layer "F.Cu") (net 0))
 (segment (start 126.7 78.5) (end 128.2 78.5) (width 0.5) (layer "F.Cu") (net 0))
 (segment (start 128.2 72.03) (end 128.73 71.5) (width 0.5) (layer "F.Cu") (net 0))
 (segment (start 118.57 98.33) (end 118.57 100.5) (width 0.5) (layer "F.Cu") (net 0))
 (segment (start 111.31 74.4) (end 108.41 71.5) (width 0.5) (layer "F.Cu") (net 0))
 (segment (start 126.7 83.5) (end 116 72.8) (width 0.5) (layer "F.Cu") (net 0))
 (segment (start 144.1 99.2) (end 145.21 99.2) (width 0.5) (layer "F.Cu") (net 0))
 (segment (start 115.61005 99.3) (end 114.69 99.3) (width 0.5) (layer "F.Cu") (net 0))
 (segment (start 161 97) (end 165 97) (width 1) (layer "F.Cu") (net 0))
 (segment (start 146.5 78.5) (end 153.5 78.5) (width 1) (layer "F.Cu") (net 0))
 (segment (start 116.03 71.83) (end 126.7 82.5) (width 0.5) (layer "F.Cu") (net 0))
 (segment (start 141.43 73.37) (end 141.43 71.5) (width 0.5) (layer "F.Cu") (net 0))
 (segment (start 111.21 97.7) (end 108.41 100.5) (width 0.5) (layer "F.Cu") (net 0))
 (segment (start 131.8 85.5) (end 133.7 85.5) (width 0.5) (layer "F.Cu") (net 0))
 (segment (start 114.69 99.3) (end 113.49 100.5) (width 0.5) (layer "F.Cu") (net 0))
 (segment (start 115 97.7) (end 111.21 97.7) (width 0.5) (layer "F.Cu") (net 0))
 (segment (start 165 75) (end 165 86) (width 3) (layer "F.Cu") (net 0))
 (segment (start 133.3 79.5) (end 136.35 76.45) (width 0.5) (layer "F.Cu") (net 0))
 (segment (start 126.6 84.5) (end 128.2 84.5) (width 0.5) (layer "F.Cu") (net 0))
 (segment (start 126.8 93.5) (end 126.19 94.11) (width 0.5) (layer "F.Cu") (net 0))
 (segment (start 123.65 76.45) (end 126.7 79.5) (width 0.5) (layer "F.Cu") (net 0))
 (segment (start 126.7 79.5) (end 128.3 79.5) (width 0.5) (layer "F.Cu") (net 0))
 (segment (start 131.8 87.5) (end 133.5 87.5) (width 0.5) (layer "F.Cu") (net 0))
 (segment (start 95 75) (end 95 97) (width 3) (layer "F.Cu") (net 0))
 (segment (start 138.89 97.09) (end 138.89 100.5) (width 0.5) (layer "F.Cu") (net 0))
 (segment (start 133.81 94.01) (end 133.81 100.5) (width 0.5) (layer "F.Cu") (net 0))
 (segment (start 126.7 81.5) (end 128.2 81.5) (width 0.5) (layer "F.Cu") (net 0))
 (segment (start 141.43 98.63) (end 141.43 100.5) (width 0.5) (layer "F.Cu") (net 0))
 (segment (start 133.3 91.5) (end 138.89 97.09) (width 0.5) (layer "F.Cu") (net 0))
 (segment (start 144.9 74.4) (end 148.69 74.4) (width 0.5) (layer "F.Cu") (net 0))
 (segment (start 118.57 71.5) (end 118.57 73.37) (width 0.5) (layer "F.Cu") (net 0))
 (segment (start 128.2 99.97) (end 128.73 100.5) (width 0.5) (layer "F.Cu") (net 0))
 (segment (start 126.7 82.5) (end 128.2 82.5) (width 0.5) (layer "F.Cu") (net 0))
 (segment (start 128.2 94.5) (end 128.2 99.97) (width 0.5) (layer "F.Cu") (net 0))
 (segment (start 126.4 92.5) (end 123.65 95.25) (width 0.5) (layer "F.Cu") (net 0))
 (segment (start 113.5 93.5) (end 115.5 91.5) (width 1) (layer "F.Cu") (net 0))
 (segment (start 146.5 93.5) (end 153.5 93.5) (width 1) (layer "F.Cu") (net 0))
 (segment (start 133.3 78.5) (end 133.81 77.99) (width 0.5) (layer "F.Cu") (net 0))
 (segment (start 133.3 89.5) (end 141.8 98) (width 0.5) (layer "F.Cu") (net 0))
 (segment (start 131.8 93.5) (end 133.3 93.5) (width 0.5) (layer "F.Cu") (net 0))
 (segment (start 133.6 83.5) (end 144.3 72.8) (width 0.5) (layer "F.Cu") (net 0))
 (segment (start 144.7 97.6) (end 148.69 97.6) (width 0.5) (layer "F.Cu") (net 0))
 (segment (start 131.8 82.5) (end 133.4 82.5) (width 0.5) (layer "F.Cu") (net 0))
 (segment (start 131.8 92.5) (end 133.3 92.5) (width 0.5) (layer "F.Cu") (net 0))
 (segment (start 114.5 73.6) (end 113.05 73.6) (width 0.5) (layer "F.Cu") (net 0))
 (segment (start 131.8 86.5) (end 133.6 86.5) (width 0.5) (layer "F.Cu") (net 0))
 (segment (start 131.8 79.5) (end 133.3 79.5) (width 0.5) (layer "F.Cu") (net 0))
 (segment (start 128.2 89.5) (end 126.4 89.5) (width 0.5) (layer "F.Cu") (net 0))
 (segment (start 126.4 89.5) (end 116.03 99.87) (width 0.5) (layer "F.Cu") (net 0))
 (segment (start 131.8 90.5) (end 133.3 90.5) (width 0.5) (layer "F.Cu") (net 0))
 (segment (start 128.2 92.5) (end 126.4 92.5) (width 0.5) (layer "F.Cu") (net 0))
 (segment (start 126.4 85.5) (end 128.2 85.5) (width 0.5) (layer "F.Cu") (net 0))
 (segment (start 133.3 80.5) (end 138.89 74.91) (width 0.5) (layer "F.Cu") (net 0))
 (segment (start 165 86) (end 165 97) (width 3) (layer "F.Cu") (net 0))
 (segment (start 153.5 78.5) (end 155.5 80.5) (width 1) (layer "F.Cu") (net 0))
 (segment (start 136.35 76.45) (end 136.35 71.5) (width 0.5) (layer "F.Cu") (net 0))
 (segment (start 128.2 90.5) (end 126.4 90.5) (width 0.5) (layer "F.Cu") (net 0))
 (segment (start 133.4 88.5) (end 144.1 99.2) (width 0.5) (layer "F.Cu") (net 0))
 (segment (start 126.2 86.5) (end 115 97.7) (width 0.5) (layer "F.Cu") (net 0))
 (segment (start 128.2 86.5) (end 126.2 86.5) (width 0.5) (layer "F.Cu") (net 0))
 (segment (start 148.69 97.6) (end 151.59 100.5) (width 0.5) (layer "F.Cu") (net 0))
 (segment (start 106.5 93.5) (end 113.5 93.5) (width 1) (layer "F.Cu") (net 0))
 (segment (start 121.11 96.79) (end 121.11 100.5) (width 0.5) (layer "F.Cu") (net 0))
 (segment (start 146.95 73.6) (end 149.05 71.5) (width 0.5) (layer "F.Cu") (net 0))
 (segment (start 131.8 94.5) (end 131.8 99.97) (width 0.5) (layer "F.Cu") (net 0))
 (segment (start 133.5 87.5) (end 144.4 98.4) (width 0.5) (layer "F.Cu") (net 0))
 (segment (start 131.8 72.03) (end 131.27 71.5) (width 0.5) (layer "F.Cu") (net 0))
 (segment (start 99 97) (end 95 97) (width 1) (layer "F.Cu") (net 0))
 (segment (start 138.89 74.91) (end 138.89 71.5) (width 0.5) (layer "F.Cu") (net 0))
 (segment (start 131.8 89.5) (end 133.3 89.5) (width 0.5) (layer "F.Cu") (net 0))
 (segment (start 126.6 84.5) (end 115.7 73.6) (width 0.5) (layer "F.Cu") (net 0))
 (segment (start 133.8 85.5) (end 144.9 74.4) (width 0.5) (layer "F.Cu") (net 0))
 (segment (start 126.4 91.5) (end 121.11 96.79) (width 0.5) (layer "F.Cu") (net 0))
 (segment (start 128.2 88.5) (end 126.41005 88.5) (width 0.5) (layer "F.Cu") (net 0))
 (segment (start 133.7 85.5) (end 133.8 85.5) (width 0.5) (layer "F.Cu") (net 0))
 (segment (start 148.69 74.4) (end 151.59 71.5) (width 0.5) (layer "F.Cu") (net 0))
 (segment (start 133.3 81.5) (end 141.43 73.37) (width 0.5) (layer "F.Cu") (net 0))
 (segment (start 145.21 72.8) (end 146.51 71.5) (width 0.5) (layer "F.Cu") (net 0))
 (segment (start 126.41005 88.5) (end 115.61005 99.3) (width 0.5) (layer "F.Cu") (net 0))
 (segment (start 144.6 73.6) (end 146.95 73.6) (width 0.5) (layer "F.Cu") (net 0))
 (segment (start 133.6 84.5) (end 133.7 84.5) (width 0.5) (layer "F.Cu") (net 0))
 (segment (start 133.81 77.99) (end 133.81 71.5) (width 0.5) (layer "F.Cu") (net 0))
 (segment (start 133.7 84.5) (end 144.6 73.6) (width 0.5) (layer "F.Cu") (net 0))
 (segment (start 159.5 80.5) (end 165 75) (width 1) (layer "F.Cu") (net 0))
 (segment (start 131.8 88.5) (end 133.4 88.5) (width 0.5) (layer "F.Cu") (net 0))
 (segment (start 115.3 98.5) (end 112.95 98.5) (width 0.5) (layer "F.Cu") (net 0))
 (segment (start 144.3 72.8) (end 145.21 72.8) (width 0.5) (layer "F.Cu") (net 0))
 (segment (start 144.4 98.4) (end 146.95 98.4) (width 0.5) (layer "F.Cu") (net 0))
 (segment (start 155.5 91.5) (end 161 97) (width 1) (layer "F.Cu") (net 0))
 (segment (start 126.19 77.99) (end 126.7 78.5) (width 0.5) (layer "F.Cu") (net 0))
 (segment (start 104.5 91.5) (end 99 97) (width 1) (layer "F.Cu") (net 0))
 (segment (start 126.19 71.5) (end 126.19 77.99) (width 0.5) (layer "F.Cu") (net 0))
 (segment (start 133.3 90.5) (end 141.43 98.63) (width 0.5) (layer "F.Cu") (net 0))
 (segment (start 131.8 99.97) (end 131.27 100.5) (width 0.5) (layer "F.Cu") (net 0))
 (segment (start 128.2 77.5) (end 128.2 72.03) (width 0.5) (layer "F.Cu") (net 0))
 (segment (start 113.5 78.5) (end 106.5 78.5) (width 1) (layer "F.Cu") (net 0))
 (segment (start 113.05 73.6) (end 110.95 71.5) (width 0.5) (layer "F.Cu") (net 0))
 (segment (start 153.5 93.5) (end 155.5 91.5) (width 1) (layer "F.Cu") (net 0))
 (segment (start 133.3 92.5) (end 136.35 95.55) (width 0.5) (layer "F.Cu") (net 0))
 (segment (start 131.8 91.5) (end 133.3 91.5) (width 0.5) (layer "F.Cu") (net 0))
 (segment (start 143.97 71.93) (end 143.97 71.5) (width 0.5) (layer "F.Cu") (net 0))
 (segment (start 112.95 98.5) (end 110.95 100.5) (width 0.5) (layer "F.Cu") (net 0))
 (segment (start 118.57 73.37) (end 126.7 81.5) (width 0.5) (layer "F.Cu") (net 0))
 (segment (start 126.19 94.11) (end 126.19 100.5) (width 0.5) (layer "F.Cu") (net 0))
 (segment (start 116.03 99.87) (end 116.03 100.5) (width 0.5) (layer "F.Cu") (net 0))
 (segment (start 141.8 98) (end 143.97 100.17) (width 0.5) (layer "F.Cu") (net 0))
 (segment (start 128.2 91.5) (end 126.4 91.5) (width 0.5) (layer "F.Cu") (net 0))
 (segment (start 144.5 91.5) (end 146.5 93.5) (width 1) (layer "F.Cu") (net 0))
 (segment (start 131.8 81.5) (end 133.3 81.5) (width 0.5) (layer "F.Cu") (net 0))
 (segment (start 104.5 80.5) (end 100.5 80.5) (width 1) (layer "F.Cu") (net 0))
 (segment (start 116.03 71.5) (end 116.03 71.83) (width 0.5) (layer "F.Cu") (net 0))
 (segment (start 131.8 84.5) (end 133.6 84.5) (width 0.5) (layer "F.Cu") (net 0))
 (segment (start 128.2 93.5) (end 126.8 93.5) (width 0.5) (layer "F.Cu") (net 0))
 (segment (start 115.5 80.5) (end 113.5 78.5) (width 1) (layer "F.Cu") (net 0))
 (segment (start 155.5 80.5) (end 159.5 80.5) (width 1) (layer "F.Cu") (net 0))
 (segment (start 131.8 80.5) (end 133.3 80.5) (width 0.5) (layer "F.Cu") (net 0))
 (segment (start 123.65 95.25) (end 123.65 100.5) (width 0.5) (layer "F.Cu") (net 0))
 (segment (start 143.97 100.17) (end 143.97 100.5) (width 0.5) (layer "F.Cu") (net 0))
 (segment (start 128.2 83.5) (end 126.7 83.5) (width 0.5) (layer "F.Cu") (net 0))
 (segment (start 126.7 80.5) (end 128.2 80.5) (width 0.5) (layer "F.Cu") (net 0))
 (segment (start 116 72.8) (end 114.79 72.8) (width 0.5) (layer "F.Cu") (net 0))
 (segment (start 126.4 85.5) (end 115.3 74.4) (width 0.5) (layer "F.Cu") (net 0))
 (segment (start 144.5 80.5) (end 146.5 78.5) (width 1) (layer "F.Cu") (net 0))
 (segment (start 106.5 78.5) (end 104.5 80.5) (width 1) (layer "F.Cu") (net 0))
 (segment (start 104.5 91.5) (end 106.5 93.5) (width 1) (layer "F.Cu") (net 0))
 (segment (start 133.6 86.5) (end 144.7 97.6) (width 0.5) (layer "F.Cu") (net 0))
 (segment (start 126.3 87.5) (end 115.3 98.5) (width 0.5) (layer "F.Cu") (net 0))
 (segment (start 128.2 87.5) (end 126.3 87.5) (width 0.5) (layer "F.Cu") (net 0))
 (segment (start 121.11 74.91) (end 126.7 80.5) (width 0.5) (layer "F.Cu") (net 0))
 (segment (start 145.21 99.2) (end 146.51 100.5) (width 0.5) (layer "F.Cu") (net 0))
 (segment (start 146.95 98.4) (end 149.05 100.5) (width 0.5) (layer "F.Cu") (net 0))
 (segment (start 123.65 71.5) (end 123.65 76.45) (width 0.5) (layer "F.Cu") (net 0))
 (segment (start 121.11 71.5) (end 121.11 74.91) (width 0.5) (layer "F.Cu") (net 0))
 (segment (start 115.7 73.6) (end 114.5 73.6) (width 0.5) (layer "F.Cu") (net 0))
 (segment (start 133.3 93.5) (end 133.81 94.01) (width 0.5) (layer "F.Cu") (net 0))
 (segment (start 115.3 74.4) (end 111.31 74.4) (width 0.5) (layer "F.Cu") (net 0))
 (segment (start 100.5 80.5) (end 95 75) (width 1) (layer "F.Cu") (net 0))
 (segment (start 114.79 72.8) (end 113.49 71.5) (width 0.5) (layer "F.Cu") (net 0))
 (segment (start 131.8 77.5) (end 131.8 72.03) (width 0.5) (layer "F.Cu") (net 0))
 (segment (start 126.4 90.5) (end 118.57 98.33) (width 0.5) (layer "F.Cu") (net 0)))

